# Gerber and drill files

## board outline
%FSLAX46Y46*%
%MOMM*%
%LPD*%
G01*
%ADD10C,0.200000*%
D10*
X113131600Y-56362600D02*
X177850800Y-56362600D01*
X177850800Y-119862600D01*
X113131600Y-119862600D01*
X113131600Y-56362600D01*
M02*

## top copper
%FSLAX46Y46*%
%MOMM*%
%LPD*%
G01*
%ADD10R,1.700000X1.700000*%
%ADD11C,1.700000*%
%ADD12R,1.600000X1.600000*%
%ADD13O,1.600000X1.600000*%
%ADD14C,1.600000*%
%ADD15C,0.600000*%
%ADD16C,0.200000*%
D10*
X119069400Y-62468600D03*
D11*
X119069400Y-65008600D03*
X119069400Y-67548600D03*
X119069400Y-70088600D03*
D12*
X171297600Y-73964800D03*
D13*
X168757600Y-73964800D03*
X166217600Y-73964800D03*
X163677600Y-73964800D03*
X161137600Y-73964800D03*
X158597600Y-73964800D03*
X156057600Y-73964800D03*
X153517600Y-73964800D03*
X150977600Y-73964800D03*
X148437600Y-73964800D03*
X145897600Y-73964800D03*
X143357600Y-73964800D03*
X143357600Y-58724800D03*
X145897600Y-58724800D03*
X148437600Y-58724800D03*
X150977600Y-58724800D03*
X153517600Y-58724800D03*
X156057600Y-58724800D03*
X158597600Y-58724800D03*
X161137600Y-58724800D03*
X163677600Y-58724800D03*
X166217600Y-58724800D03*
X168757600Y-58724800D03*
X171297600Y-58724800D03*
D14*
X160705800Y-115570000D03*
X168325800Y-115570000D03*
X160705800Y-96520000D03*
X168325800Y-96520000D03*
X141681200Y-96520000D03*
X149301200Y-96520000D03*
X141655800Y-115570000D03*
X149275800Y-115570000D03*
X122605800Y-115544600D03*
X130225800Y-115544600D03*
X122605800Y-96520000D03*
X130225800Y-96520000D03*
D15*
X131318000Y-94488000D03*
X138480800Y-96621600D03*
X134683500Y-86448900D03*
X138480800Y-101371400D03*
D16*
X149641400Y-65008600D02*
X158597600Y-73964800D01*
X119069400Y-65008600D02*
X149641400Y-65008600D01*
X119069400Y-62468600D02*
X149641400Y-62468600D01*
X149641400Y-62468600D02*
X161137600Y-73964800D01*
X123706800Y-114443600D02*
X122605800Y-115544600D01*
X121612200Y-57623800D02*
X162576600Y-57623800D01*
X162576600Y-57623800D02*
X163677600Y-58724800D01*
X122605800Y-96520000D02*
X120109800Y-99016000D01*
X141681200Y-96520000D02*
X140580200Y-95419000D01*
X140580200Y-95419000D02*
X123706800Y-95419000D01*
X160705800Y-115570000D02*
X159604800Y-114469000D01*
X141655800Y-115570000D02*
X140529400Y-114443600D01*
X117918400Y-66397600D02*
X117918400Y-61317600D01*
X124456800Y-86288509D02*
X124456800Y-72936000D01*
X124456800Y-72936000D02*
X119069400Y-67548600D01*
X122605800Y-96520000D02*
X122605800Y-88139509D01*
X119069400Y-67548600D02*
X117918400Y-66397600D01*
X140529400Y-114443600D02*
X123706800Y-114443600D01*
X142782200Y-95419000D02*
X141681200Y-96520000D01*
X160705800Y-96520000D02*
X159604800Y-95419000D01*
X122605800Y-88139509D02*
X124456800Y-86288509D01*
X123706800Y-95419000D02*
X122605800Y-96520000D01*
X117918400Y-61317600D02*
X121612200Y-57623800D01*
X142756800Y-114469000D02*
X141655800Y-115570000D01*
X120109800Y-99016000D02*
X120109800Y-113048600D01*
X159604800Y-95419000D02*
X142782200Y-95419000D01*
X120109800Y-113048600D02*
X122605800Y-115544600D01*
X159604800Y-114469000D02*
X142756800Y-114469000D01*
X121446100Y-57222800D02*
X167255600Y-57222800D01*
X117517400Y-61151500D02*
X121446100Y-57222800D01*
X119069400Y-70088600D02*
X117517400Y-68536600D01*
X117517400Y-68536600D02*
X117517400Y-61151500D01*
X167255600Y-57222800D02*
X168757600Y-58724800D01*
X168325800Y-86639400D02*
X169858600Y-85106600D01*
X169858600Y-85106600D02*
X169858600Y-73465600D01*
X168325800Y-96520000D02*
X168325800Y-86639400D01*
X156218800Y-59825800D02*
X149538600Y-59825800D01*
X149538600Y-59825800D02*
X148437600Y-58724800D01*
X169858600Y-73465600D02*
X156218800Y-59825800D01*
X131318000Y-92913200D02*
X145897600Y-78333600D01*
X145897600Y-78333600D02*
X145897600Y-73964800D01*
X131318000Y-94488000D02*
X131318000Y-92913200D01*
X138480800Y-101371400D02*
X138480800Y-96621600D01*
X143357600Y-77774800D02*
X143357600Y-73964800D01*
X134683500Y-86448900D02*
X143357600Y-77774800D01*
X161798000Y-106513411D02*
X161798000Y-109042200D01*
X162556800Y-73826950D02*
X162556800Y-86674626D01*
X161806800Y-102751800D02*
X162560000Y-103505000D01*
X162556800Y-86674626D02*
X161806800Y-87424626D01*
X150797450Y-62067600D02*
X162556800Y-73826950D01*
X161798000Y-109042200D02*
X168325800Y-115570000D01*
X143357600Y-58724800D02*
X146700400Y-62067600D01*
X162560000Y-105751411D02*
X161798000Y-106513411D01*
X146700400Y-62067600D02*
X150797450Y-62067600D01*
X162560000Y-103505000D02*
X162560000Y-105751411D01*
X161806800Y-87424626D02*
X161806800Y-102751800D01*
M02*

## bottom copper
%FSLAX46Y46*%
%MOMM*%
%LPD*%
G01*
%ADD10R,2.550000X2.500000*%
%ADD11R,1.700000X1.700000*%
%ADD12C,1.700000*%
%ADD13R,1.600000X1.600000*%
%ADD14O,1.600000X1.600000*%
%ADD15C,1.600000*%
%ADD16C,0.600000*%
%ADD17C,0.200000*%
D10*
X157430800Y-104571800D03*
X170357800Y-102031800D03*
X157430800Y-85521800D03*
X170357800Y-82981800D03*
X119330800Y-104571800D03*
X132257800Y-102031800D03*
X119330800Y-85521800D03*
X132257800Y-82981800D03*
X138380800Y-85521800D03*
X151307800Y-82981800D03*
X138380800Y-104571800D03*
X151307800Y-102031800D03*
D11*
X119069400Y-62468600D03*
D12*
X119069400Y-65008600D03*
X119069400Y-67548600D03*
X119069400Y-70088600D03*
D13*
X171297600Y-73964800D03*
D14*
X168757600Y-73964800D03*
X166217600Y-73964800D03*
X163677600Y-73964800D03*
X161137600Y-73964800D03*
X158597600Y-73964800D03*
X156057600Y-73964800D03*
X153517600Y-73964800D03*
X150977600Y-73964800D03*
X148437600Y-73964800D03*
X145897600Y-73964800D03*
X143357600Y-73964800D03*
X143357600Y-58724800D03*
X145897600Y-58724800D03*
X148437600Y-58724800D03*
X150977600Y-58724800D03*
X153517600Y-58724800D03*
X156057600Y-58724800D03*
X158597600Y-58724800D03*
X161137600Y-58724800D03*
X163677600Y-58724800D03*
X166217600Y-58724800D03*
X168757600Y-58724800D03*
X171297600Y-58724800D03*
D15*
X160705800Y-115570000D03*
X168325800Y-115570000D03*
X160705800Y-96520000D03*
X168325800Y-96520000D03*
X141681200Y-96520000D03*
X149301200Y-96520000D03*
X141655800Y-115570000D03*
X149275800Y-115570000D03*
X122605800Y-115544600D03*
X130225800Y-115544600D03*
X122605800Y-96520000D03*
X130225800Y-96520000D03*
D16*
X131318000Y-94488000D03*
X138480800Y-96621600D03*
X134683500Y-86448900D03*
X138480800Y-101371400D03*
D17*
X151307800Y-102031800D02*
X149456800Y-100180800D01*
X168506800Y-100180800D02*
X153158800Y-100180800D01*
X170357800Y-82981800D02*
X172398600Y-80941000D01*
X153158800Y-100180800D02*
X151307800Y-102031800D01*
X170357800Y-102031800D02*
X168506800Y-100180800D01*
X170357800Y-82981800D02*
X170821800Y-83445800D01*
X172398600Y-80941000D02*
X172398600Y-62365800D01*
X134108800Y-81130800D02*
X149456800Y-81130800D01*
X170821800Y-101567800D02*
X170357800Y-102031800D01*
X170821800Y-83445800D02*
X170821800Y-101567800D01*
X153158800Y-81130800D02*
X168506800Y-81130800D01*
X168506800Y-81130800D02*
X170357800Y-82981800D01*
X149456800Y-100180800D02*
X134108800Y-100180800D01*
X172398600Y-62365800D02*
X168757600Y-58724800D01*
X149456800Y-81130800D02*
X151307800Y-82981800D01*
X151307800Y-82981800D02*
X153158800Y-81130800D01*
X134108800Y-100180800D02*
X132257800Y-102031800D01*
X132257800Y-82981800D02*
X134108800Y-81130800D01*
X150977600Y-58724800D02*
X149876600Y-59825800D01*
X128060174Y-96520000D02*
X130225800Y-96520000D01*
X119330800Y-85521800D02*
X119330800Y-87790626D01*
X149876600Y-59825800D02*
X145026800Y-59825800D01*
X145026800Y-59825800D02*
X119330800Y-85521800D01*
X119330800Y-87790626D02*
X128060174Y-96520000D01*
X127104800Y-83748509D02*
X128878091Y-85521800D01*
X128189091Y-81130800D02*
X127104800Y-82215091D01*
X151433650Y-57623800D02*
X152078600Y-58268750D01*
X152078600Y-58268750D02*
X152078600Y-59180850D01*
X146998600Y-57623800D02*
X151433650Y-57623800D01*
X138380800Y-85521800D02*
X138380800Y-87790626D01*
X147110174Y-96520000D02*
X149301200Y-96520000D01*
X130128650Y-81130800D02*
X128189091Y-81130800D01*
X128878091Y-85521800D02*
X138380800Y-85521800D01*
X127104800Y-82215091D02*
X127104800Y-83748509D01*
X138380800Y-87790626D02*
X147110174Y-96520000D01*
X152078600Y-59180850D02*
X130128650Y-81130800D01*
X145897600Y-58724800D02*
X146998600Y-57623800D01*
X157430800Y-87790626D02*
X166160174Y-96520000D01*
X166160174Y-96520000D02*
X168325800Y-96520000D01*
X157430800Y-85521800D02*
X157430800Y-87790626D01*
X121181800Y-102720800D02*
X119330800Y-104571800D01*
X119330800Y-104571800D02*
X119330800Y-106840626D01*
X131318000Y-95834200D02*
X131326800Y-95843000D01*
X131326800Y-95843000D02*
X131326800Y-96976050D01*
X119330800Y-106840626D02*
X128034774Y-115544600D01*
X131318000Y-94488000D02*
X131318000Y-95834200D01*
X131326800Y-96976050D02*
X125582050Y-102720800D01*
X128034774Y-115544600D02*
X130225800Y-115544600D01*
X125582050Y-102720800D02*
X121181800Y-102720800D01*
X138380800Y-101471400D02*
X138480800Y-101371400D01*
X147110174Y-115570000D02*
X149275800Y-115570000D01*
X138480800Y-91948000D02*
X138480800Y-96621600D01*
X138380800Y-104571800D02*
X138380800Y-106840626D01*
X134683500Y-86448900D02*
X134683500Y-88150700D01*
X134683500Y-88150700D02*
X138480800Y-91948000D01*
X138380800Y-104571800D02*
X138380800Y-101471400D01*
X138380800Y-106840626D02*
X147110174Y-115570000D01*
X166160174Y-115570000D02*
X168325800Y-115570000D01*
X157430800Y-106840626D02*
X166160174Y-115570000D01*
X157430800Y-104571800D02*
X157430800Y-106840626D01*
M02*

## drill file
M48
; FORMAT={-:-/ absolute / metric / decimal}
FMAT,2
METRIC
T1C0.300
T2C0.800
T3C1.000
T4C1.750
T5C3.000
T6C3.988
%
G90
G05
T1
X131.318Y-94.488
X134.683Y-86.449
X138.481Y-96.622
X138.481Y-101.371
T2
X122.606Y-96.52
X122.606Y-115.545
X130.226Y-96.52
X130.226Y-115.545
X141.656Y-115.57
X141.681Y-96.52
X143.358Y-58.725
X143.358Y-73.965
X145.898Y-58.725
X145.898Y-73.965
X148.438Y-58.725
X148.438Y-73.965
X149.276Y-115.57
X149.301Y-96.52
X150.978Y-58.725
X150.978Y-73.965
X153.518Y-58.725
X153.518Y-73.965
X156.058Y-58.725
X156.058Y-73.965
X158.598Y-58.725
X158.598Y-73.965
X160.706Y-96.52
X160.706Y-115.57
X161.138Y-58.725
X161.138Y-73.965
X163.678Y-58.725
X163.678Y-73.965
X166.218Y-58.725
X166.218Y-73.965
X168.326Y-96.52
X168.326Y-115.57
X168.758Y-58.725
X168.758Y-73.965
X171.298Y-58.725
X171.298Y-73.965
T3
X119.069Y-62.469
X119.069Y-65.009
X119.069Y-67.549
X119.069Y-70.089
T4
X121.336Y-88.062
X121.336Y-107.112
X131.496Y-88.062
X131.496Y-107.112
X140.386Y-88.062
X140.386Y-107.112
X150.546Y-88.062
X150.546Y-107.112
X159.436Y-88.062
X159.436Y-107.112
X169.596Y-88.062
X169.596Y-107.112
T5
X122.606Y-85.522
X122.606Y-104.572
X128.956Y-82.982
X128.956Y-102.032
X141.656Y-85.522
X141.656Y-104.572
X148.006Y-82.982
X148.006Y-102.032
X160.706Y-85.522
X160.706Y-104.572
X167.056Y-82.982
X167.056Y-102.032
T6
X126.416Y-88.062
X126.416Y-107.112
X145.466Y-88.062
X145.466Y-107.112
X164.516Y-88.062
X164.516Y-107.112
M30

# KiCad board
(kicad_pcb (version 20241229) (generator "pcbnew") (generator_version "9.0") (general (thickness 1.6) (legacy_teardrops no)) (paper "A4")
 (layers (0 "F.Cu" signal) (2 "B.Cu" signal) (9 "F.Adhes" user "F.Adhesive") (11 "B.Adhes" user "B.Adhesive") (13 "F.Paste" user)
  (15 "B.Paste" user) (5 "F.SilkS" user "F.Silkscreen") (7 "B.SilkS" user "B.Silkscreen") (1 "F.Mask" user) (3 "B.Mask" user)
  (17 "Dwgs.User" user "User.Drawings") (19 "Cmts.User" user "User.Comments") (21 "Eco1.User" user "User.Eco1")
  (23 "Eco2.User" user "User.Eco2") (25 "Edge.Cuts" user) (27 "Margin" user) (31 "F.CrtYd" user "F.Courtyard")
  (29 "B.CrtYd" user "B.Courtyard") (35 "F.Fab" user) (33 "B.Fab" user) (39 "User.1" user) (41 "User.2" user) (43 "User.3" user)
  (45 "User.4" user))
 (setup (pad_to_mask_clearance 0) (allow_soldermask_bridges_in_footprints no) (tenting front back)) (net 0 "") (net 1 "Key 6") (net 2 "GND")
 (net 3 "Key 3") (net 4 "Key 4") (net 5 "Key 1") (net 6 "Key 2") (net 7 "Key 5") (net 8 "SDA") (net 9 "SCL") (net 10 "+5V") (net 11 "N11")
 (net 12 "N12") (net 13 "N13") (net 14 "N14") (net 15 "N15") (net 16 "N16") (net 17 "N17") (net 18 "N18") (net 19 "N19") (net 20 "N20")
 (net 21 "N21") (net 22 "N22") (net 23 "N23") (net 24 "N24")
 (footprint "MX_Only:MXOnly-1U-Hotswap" (layer "F.Cu") (at 164.5158 107.1118)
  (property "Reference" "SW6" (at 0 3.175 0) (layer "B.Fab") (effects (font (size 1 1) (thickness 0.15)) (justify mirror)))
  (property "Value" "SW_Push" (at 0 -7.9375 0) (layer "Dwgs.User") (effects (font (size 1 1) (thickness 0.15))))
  (pad "" np_thru_hole circle (at -5.08 0 48.0996) (size 1.75 1.75) (drill 1.75) (layers "*.Cu" "*.Mask"))
  (pad "" np_thru_hole circle (at -3.81 -2.54) (size 3 3) (drill 3) (layers "*.Cu" "*.Mask"))
  (pad "" np_thru_hole circle (at 0 0) (size 3.9878 3.9878) (drill 3.9878) (layers "*.Cu" "*.Mask"))
  (pad "" np_thru_hole circle (at 2.54 -5.08) (size 3 3) (drill 3) (layers "*.Cu" "*.Mask"))
  (pad "" np_thru_hole circle (at 5.08 0 48.0996) (size 1.75 1.75) (drill 1.75) (layers "*.Cu" "*.Mask"))
  (pad "1" smd rect (at -7.085 -2.54) (size 2.55 2.5) (layers "B.Cu" "B.Mask" "B.Paste") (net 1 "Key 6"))
  (pad "2" smd rect (at 5.842 -5.08) (size 2.55 2.5) (layers "B.Cu" "B.Mask" "B.Paste") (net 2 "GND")))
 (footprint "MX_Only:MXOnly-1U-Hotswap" (layer "F.Cu") (at 164.5158 88.0618)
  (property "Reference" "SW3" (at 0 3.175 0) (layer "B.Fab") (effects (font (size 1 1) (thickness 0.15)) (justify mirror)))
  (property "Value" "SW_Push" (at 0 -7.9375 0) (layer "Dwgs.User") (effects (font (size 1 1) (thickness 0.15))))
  (pad "" np_thru_hole circle (at -5.08 0 48.0996) (size 1.75 1.75) (drill 1.75) (layers "*.Cu" "*.Mask"))
  (pad "" np_thru_hole circle (at -3.81 -2.54) (size 3 3) (drill 3) (layers "*.Cu" "*.Mask"))
  (pad "" np_thru_hole circle (at 0 0) (size 3.9878 3.9878) (drill 3.9878) (layers "*.Cu" "*.Mask"))
  (pad "" np_thru_hole circle (at 2.54 -5.08) (size 3 3) (drill 3) (layers "*.Cu" "*.Mask"))
  (pad "" np_thru_hole circle (at 5.08 0 48.0996) (size 1.75 1.75) (drill 1.75) (layers "*.Cu" "*.Mask"))
  (pad "1" smd rect (at -7.085 -2.54) (size 2.55 2.5) (layers "B.Cu" "B.Mask" "B.Paste") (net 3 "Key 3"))
  (pad "2" smd rect (at 5.842 -5.08) (size 2.55 2.5) (layers "B.Cu" "B.Mask" "B.Paste") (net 2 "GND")))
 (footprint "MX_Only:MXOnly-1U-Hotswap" (layer "F.Cu") (at 126.4158 107.1118)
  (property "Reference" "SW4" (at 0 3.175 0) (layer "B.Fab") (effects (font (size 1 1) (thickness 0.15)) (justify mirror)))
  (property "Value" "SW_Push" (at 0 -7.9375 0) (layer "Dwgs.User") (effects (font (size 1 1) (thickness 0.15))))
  (pad "" np_thru_hole circle (at -5.08 0 48.0996) (size 1.75 1.75) (drill 1.75) (layers "*.Cu" "*.Mask"))
  (pad "" np_thru_hole circle (at -3.81 -2.54) (size 3 3) (drill 3) (layers "*.Cu" "*.Mask"))
  (pad "" np_thru_hole circle (at 0 0) (size 3.9878 3.9878) (drill 3.9878) (layers "*.Cu" "*.Mask"))
  (pad "" np_thru_hole circle (at 2.54 -5.08) (size 3 3) (drill 3) (layers "*.Cu" "*.Mask"))
  (pad "" np_thru_hole circle (at 5.08 0 48.0996) (size 1.75 1.75) (drill 1.75) (layers "*.Cu" "*.Mask"))
  (pad "1" smd rect (at -7.085 -2.54) (size 2.55 2.5) (layers "B.Cu" "B.Mask" "B.Paste") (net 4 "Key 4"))
  (pad "2" smd rect (at 5.842 -5.08) (size 2.55 2.5) (layers "B.Cu" "B.Mask" "B.Paste") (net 2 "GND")))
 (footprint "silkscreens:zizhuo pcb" (layer "F.Cu") (at 164.6936 67.346207 90)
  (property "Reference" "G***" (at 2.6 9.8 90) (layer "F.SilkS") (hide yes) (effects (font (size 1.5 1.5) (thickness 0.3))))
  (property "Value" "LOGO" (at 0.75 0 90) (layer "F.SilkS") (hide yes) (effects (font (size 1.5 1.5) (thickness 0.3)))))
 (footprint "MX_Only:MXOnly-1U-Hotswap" (layer "F.Cu") (at 126.4158 88.0618)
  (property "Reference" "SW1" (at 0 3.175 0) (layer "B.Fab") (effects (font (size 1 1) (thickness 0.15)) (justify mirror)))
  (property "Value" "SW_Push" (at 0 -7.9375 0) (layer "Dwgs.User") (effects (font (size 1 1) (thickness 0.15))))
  (pad "" np_thru_hole circle (at -5.08 0 48.0996) (size 1.75 1.75) (drill 1.75) (layers "*.Cu" "*.Mask"))
  (pad "" np_thru_hole circle (at -3.81 -2.54) (size 3 3) (drill 3) (layers "*.Cu" "*.Mask"))
  (pad "" np_thru_hole circle (at 0 0) (size 3.9878 3.9878) (drill 3.9878) (layers "*.Cu" "*.Mask"))
  (pad "" np_thru_hole circle (at 2.54 -5.08) (size 3 3) (drill 3) (layers "*.Cu" "*.Mask"))
  (pad "" np_thru_hole circle (at 5.08 0 48.0996) (size 1.75 1.75) (drill 1.75) (layers "*.Cu" "*.Mask"))
  (pad "1" smd rect (at -7.085 -2.54) (size 2.55 2.5) (layers "B.Cu" "B.Mask" "B.Paste") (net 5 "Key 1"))
  (pad "2" smd rect (at 5.842 -5.08) (size 2.55 2.5) (layers "B.Cu" "B.Mask" "B.Paste") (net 2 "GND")))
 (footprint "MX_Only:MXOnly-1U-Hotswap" (layer "F.Cu") (at 145.4658 88.0618)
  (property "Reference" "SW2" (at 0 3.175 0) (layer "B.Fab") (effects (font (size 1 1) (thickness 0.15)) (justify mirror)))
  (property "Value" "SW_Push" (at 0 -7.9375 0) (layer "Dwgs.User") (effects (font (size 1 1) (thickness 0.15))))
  (pad "" np_thru_hole circle (at -5.08 0 48.0996) (size 1.75 1.75) (drill 1.75) (layers "*.Cu" "*.Mask"))
  (pad "" np_thru_hole circle (at -3.81 -2.54) (size 3 3) (drill 3) (layers "*.Cu" "*.Mask"))
  (pad "" np_thru_hole circle (at 0 0) (size 3.9878 3.9878) (drill 3.9878) (layers "*.Cu" "*.Mask"))
  (pad "" np_thru_hole circle (at 2.54 -5.08) (size 3 3) (drill 3) (layers "*.Cu" "*.Mask"))
  (pad "" np_thru_hole circle (at 5.08 0 48.0996) (size 1.75 1.75) (drill 1.75) (layers "*.Cu" "*.Mask"))
  (pad "1" smd rect (at -7.085 -2.54) (size 2.55 2.5) (layers "B.Cu" "B.Mask" "B.Paste") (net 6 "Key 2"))
  (pad "2" smd rect (at 5.842 -5.08) (size 2.55 2.5) (layers "B.Cu" "B.Mask" "B.Paste") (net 2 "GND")))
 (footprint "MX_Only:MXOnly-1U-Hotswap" (layer "F.Cu") (at 145.4658 107.1118)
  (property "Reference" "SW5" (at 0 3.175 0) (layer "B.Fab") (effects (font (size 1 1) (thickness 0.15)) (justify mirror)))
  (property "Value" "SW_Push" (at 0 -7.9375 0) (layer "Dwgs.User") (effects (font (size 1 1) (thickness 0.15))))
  (pad "" np_thru_hole circle (at -5.08 0 48.0996) (size 1.75 1.75) (drill 1.75) (layers "*.Cu" "*.Mask"))
  (pad "" np_thru_hole circle (at -3.81 -2.54) (size 3 3) (drill 3) (layers "*.Cu" "*.Mask"))
  (pad "" np_thru_hole circle (at 0 0) (size 3.9878 3.9878) (drill 3.9878) (layers "*.Cu" "*.Mask"))
  (pad "" np_thru_hole circle (at 2.54 -5.08) (size 3 3) (drill 3) (layers "*.Cu" "*.Mask"))
  (pad "" np_thru_hole circle (at 5.08 0 48.0996) (size 1.75 1.75) (drill 1.75) (layers "*.Cu" "*.Mask"))
  (pad "1" smd rect (at -7.085 -2.54) (size 2.55 2.5) (layers "B.Cu" "B.Mask" "B.Paste") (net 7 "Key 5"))
  (pad "2" smd rect (at 5.842 -5.08) (size 2.55 2.5) (layers "B.Cu" "B.Mask" "B.Paste") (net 2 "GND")))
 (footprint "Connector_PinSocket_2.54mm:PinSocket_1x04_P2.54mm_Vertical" (layer "F.Cu") (at 119.0694 62.4686)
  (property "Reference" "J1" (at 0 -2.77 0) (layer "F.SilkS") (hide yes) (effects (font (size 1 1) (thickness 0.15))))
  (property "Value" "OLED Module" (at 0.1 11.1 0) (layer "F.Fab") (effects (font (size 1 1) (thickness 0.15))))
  (pad "1" thru_hole rect (at 0 0) (size 1.7 1.7) (drill 1) (layers "*.Cu" "*.Mask") (remove_unused_layers no) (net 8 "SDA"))
  (pad "2" thru_hole circle (at 0 2.54) (size 1.7 1.7) (drill 1) (layers "*.Cu" "*.Mask") (remove_unused_layers no) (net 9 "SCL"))
  (pad "3" thru_hole circle (at 0 5.08) (size 1.7 1.7) (drill 1) (layers "*.Cu" "*.Mask") (remove_unused_layers no) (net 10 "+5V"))
  (pad "4" thru_hole circle (at 0 7.62) (size 1.7 1.7) (drill 1) (layers "*.Cu" "*.Mask") (remove_unused_layers no) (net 2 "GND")))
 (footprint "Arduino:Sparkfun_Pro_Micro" (layer "B.Cu") (at 143.3576 58.7248 -90)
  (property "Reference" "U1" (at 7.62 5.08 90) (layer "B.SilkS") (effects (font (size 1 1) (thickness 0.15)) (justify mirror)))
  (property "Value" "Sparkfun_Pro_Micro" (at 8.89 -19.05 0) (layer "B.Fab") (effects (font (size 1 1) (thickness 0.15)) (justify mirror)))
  (pad "1" thru_hole rect (at 15.24 -27.94 270) (size 1.6 1.6) (drill 0.8) (layers "*.Cu" "*.Mask") (remove_unused_layers no) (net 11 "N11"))
  (pad "2" thru_hole oval (at 15.24 -25.4 270) (size 1.6 1.6) (drill 0.8) (layers "*.Cu" "*.Mask") (remove_unused_layers no) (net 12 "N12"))
  (pad "3" thru_hole oval (at 15.24 -22.86 270) (size 1.6 1.6) (drill 0.8) (layers "*.Cu" "*.Mask") (remove_unused_layers no) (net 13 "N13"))
  (pad "4" thru_hole oval (at 15.24 -20.32 270) (size 1.6 1.6) (drill 0.8) (layers "*.Cu" "*.Mask") (remove_unused_layers no) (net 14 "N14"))
  (pad "5" thru_hole oval (at 15.24 -17.78 270) (size 1.6 1.6) (drill 0.8) (layers "*.Cu" "*.Mask") (remove_unused_layers no) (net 8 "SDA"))
  (pad "6" thru_hole oval (at 15.24 -15.24 270) (size 1.6 1.6) (drill 0.8) (layers "*.Cu" "*.Mask") (remove_unused_layers no) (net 9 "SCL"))
  (pad "7" thru_hole oval (at 15.24 -12.7 270) (size 1.6 1.6) (drill 0.8) (layers "*.Cu" "*.Mask") (remove_unused_layers no) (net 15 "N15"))
  (pad "8" thru_hole oval (at 15.24 -10.16 270) (size 1.6 1.6) (drill 0.8) (layers "*.Cu" "*.Mask") (remove_unused_layers no) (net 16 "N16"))
  (pad "9" thru_hole oval (at 15.24 -7.62 270) (size 1.6 1.6) (drill 0.8) (layers "*.Cu" "*.Mask") (remove_unused_layers no) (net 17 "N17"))
  (pad "10" thru_hole oval (at 15.24 -5.08 270) (size 1.6 1.6) (drill 0.8) (layers "*.Cu" "*.Mask") (remove_unused_layers no) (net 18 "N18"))
  (pad "11" thru_hole oval (at 15.24 -2.54 270) (size 1.6 1.6) (drill 0.8) (layers "*.Cu" "*.Mask") (remove_unused_layers no)
   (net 4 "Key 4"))
  (pad "12" thru_hole oval (at 15.24 0 270) (size 1.6 1.6) (drill 0.8) (layers "*.Cu" "*.Mask") (remove_unused_layers no) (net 7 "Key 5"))
  (pad "13" thru_hole oval (at 0 0 270) (size 1.6 1.6) (drill 0.8) (layers "*.Cu" "*.Mask") (remove_unused_layers no) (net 1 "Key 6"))
  (pad "14" thru_hole oval (at 0 -2.54 270) (size 1.6 1.6) (drill 0.8) (layers "*.Cu" "*.Mask") (remove_unused_layers no) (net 6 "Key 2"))
  (pad "15" thru_hole oval (at 0 -5.08 270) (size 1.6 1.6) (drill 0.8) (layers "*.Cu" "*.Mask") (remove_unused_layers no) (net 3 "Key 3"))
  (pad "16" thru_hole oval (at 0 -7.62 270) (size 1.6 1.6) (drill 0.8) (layers "*.Cu" "*.Mask") (remove_unused_layers no) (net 5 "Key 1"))
  (pad "17" thru_hole oval (at 0 -10.16 270) (size 1.6 1.6) (drill 0.8) (layers "*.Cu" "*.Mask") (remove_unused_layers no) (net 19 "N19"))
  (pad "18" thru_hole oval (at 0 -12.7 270) (size 1.6 1.6) (drill 0.8) (layers "*.Cu" "*.Mask") (remove_unused_layers no) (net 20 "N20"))
  (pad "19" thru_hole oval (at 0 -15.24 270) (size 1.6 1.6) (drill 0.8) (layers "*.Cu" "*.Mask") (remove_unused_layers no) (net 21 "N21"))
  (pad "20" thru_hole oval (at 0 -17.78 270) (size 1.6 1.6) (drill 0.8) (layers "*.Cu" "*.Mask") (remove_unused_layers no) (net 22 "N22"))
  (pad "21" thru_hole oval (at 0 -20.32 270) (size 1.6 1.6) (drill 0.8) (layers "*.Cu" "*.Mask") (remove_unused_layers no) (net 10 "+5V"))
  (pad "22" thru_hole oval (at 0 -22.86 270) (size 1.6 1.6) (drill 0.8) (layers "*.Cu" "*.Mask") (remove_unused_layers no) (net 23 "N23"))
  (pad "23" thru_hole oval (at 0 -25.4 270) (size 1.6 1.6) (drill 0.8) (layers "*.Cu" "*.Mask") (remove_unused_layers no) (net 2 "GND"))
  (pad "24" thru_hole oval (at 0 -27.94 270) (size 1.6 1.6) (drill 0.8) (layers "*.Cu" "*.Mask") (remove_unused_layers no) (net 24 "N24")))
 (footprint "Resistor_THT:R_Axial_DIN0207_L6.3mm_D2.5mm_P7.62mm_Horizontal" (layer "B.Cu") (at 160.7058 115.57)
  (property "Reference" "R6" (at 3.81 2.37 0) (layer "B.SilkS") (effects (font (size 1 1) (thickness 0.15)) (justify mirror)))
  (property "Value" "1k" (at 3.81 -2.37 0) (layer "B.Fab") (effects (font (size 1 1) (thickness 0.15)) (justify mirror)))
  (pad "1" thru_hole circle (at 0 0) (size 1.6 1.6) (drill 0.8) (layers "*.Cu" "*.Mask") (remove_unused_layers no) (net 10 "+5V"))
  (pad "2" thru_hole circle (at 7.62 0) (size 1.6 1.6) (drill 0.8) (layers "*.Cu" "*.Mask") (remove_unused_layers no) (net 1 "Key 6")))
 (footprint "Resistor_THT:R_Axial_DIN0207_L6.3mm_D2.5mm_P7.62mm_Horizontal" (layer "B.Cu") (at 160.7058 96.52)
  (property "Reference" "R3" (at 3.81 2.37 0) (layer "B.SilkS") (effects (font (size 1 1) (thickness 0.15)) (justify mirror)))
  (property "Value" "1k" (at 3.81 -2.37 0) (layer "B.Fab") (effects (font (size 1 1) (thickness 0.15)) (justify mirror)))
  (pad "1" thru_hole circle (at 0 0) (size 1.6 1.6) (drill 0.8) (layers "*.Cu" "*.Mask") (remove_unused_layers no) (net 10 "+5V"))
  (pad "2" thru_hole circle (at 7.62 0) (size 1.6 1.6) (drill 0.8) (layers "*.Cu" "*.Mask") (remove_unused_layers no) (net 3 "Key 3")))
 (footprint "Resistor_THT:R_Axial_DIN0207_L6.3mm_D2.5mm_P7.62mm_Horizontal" (layer "B.Cu") (at 141.6812 96.52)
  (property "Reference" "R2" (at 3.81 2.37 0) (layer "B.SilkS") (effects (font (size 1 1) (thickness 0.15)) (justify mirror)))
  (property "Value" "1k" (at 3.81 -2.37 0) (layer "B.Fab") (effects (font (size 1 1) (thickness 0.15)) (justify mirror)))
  (pad "1" thru_hole circle (at 0 0) (size 1.6 1.6) (drill 0.8) (layers "*.Cu" "*.Mask") (remove_unused_layers no) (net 10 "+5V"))
  (pad "2" thru_hole circle (at 7.62 0) (size 1.6 1.6) (drill 0.8) (layers "*.Cu" "*.Mask") (remove_unused_layers no) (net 6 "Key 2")))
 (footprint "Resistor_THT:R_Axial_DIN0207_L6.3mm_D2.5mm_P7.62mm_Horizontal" (layer "B.Cu") (at 141.6558 115.57)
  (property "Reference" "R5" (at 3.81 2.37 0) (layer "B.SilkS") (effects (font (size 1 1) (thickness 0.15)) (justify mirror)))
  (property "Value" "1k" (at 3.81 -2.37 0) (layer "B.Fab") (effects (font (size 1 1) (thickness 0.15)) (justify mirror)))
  (pad "1" thru_hole circle (at 0 0) (size 1.6 1.6) (drill 0.8) (layers "*.Cu" "*.Mask") (remove_unused_layers no) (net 10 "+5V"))
  (pad "2" thru_hole circle (at 7.62 0) (size 1.6 1.6) (drill 0.8) (layers "*.Cu" "*.Mask") (remove_unused_layers no) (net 7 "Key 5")))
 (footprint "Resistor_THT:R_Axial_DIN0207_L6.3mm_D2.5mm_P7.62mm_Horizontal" (layer "B.Cu") (at 122.6058 115.5446)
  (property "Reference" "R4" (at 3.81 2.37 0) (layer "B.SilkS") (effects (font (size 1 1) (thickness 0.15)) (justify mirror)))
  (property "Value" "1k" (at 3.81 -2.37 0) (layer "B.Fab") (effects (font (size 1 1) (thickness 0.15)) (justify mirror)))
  (pad "1" thru_hole circle (at 0 0) (size 1.6 1.6) (drill 0.8) (layers "*.Cu" "*.Mask") (remove_unused_layers no) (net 10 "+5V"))
  (pad "2" thru_hole circle (at 7.62 0) (size 1.6 1.6) (drill 0.8) (layers "*.Cu" "*.Mask") (remove_unused_layers no) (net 4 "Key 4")))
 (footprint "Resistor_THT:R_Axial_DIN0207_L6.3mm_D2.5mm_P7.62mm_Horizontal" (layer "B.Cu") (at 122.6058 96.52)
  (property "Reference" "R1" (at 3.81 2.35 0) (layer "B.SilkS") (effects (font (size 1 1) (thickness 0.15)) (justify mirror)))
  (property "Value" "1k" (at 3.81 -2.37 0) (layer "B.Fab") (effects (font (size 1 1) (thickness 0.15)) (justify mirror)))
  (pad "1" thru_hole circle (at 0 0) (size 1.6 1.6) (drill 0.8) (layers "*.Cu" "*.Mask") (remove_unused_layers no) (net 10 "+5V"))
  (pad "2" thru_hole circle (at 7.62 0) (size 1.6 1.6) (drill 0.8) (layers "*.Cu" "*.Mask") (remove_unused_layers no) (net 5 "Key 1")))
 (gr_rect (start 113.1316 56.3626) (end 177.8508 119.8626) (stroke (width 0.2) (type solid)) (fill no) (layer "Edge.Cuts"))
 (segment (start 149.6414 65.0086) (end 158.5976 73.9648) (width 0.2) (layer "F.Cu") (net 9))
 (segment (start 119.0694 65.0086) (end 149.6414 65.0086) (width 0.2) (layer "F.Cu") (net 9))
 (segment (start 119.0694 62.4686) (end 149.6414 62.4686) (width 0.2) (layer "F.Cu") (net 8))
 (segment (start 149.6414 62.4686) (end 161.1376 73.9648) (width 0.2) (layer "F.Cu") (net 8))
 (segment (start 123.7068 114.4436) (end 122.6058 115.5446) (width 0.2) (layer "F.Cu") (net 10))
 (segment (start 121.6122 57.6238) (end 162.5766 57.6238) (width 0.2) (layer "F.Cu") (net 10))
 (segment (start 162.5766 57.6238) (end 163.6776 58.7248) (width 0.2) (layer "F.Cu") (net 10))
 (segment (start 122.6058 96.52) (end 120.1098 99.016) (width 0.2) (layer "F.Cu") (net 10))
 (segment (start 141.6812 96.52) (end 140.5802 95.419) (width 0.2) (layer "F.Cu") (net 10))
 (segment (start 140.5802 95.419) (end 123.7068 95.419) (width 0.2) (layer "F.Cu") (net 10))
 (segment (start 160.7058 115.57) (end 159.6048 114.469) (width 0.2) (layer "F.Cu") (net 10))
 (segment (start 141.6558 115.57) (end 140.5294 114.4436) (width 0.2) (layer "F.Cu") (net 10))
 (segment (start 117.9184 66.3976) (end 117.9184 61.3176) (width 0.2) (layer "F.Cu") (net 10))
 (segment (start 124.4568 86.288509) (end 124.4568 72.936) (width 0.2) (layer "F.Cu") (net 10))
 (segment (start 124.4568 72.936) (end 119.0694 67.5486) (width 0.2) (layer "F.Cu") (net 10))
 (segment (start 122.6058 96.52) (end 122.6058 88.139509) (width 0.2) (layer "F.Cu") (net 10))
 (segment (start 119.0694 67.5486) (end 117.9184 66.3976) (width 0.2) (layer "F.Cu") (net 10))
 (segment (start 140.5294 114.4436) (end 123.7068 114.4436) (width 0.2) (layer "F.Cu") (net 10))
 (segment (start 142.7822 95.419) (end 141.6812 96.52) (width 0.2) (layer "F.Cu") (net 10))
 (segment (start 160.7058 96.52) (end 159.6048 95.419) (width 0.2) (layer "F.Cu") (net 10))
 (segment (start 122.6058 88.139509) (end 124.4568 86.288509) (width 0.2) (layer "F.Cu") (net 10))
 (segment (start 123.7068 95.419) (end 122.6058 96.52) (width 0.2) (layer "F.Cu") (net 10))
 (segment (start 117.9184 61.3176) (end 121.6122 57.6238) (width 0.2) (layer "F.Cu") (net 10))
 (segment (start 142.7568 114.469) (end 141.6558 115.57) (width 0.2) (layer "F.Cu") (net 10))
 (segment (start 120.1098 99.016) (end 120.1098 113.0486) (width 0.2) (layer "F.Cu") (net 10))
 (segment (start 159.6048 95.419) (end 142.7822 95.419) (width 0.2) (layer "F.Cu") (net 10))
 (segment (start 120.1098 113.0486) (end 122.6058 115.5446) (width 0.2) (layer "F.Cu") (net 10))
 (segment (start 159.6048 114.469) (end 142.7568 114.469) (width 0.2) (layer "F.Cu") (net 10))
 (segment (start 121.4461 57.2228) (end 167.2556 57.2228) (width 0.2) (layer "F.Cu") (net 2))
 (segment (start 117.5174 61.1515) (end 121.4461 57.2228) (width 0.2) (layer "F.Cu") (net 2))
 (segment (start 119.0694 70.0886) (end 117.5174 68.5366) (width 0.2) (layer "F.Cu") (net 2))
 (segment (start 117.5174 68.5366) (end 117.5174 61.1515) (width 0.2) (layer "F.Cu") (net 2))
 (segment (start 167.2556 57.2228) (end 168.7576 58.7248) (width 0.2) (layer "F.Cu") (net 2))
 (segment (start 151.3078 102.0318) (end 149.4568 100.1808) (width 0.2) (layer "B.Cu") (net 2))
 (segment (start 168.5068 100.1808) (end 153.1588 100.1808) (width 0.2) (layer "B.Cu") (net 2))
 (segment (start 170.3578 82.9818) (end 172.3986 80.941) (width 0.2) (layer "B.Cu") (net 2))
 (segment (start 153.1588 100.1808) (end 151.3078 102.0318) (width 0.2) (layer "B.Cu") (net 2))
 (segment (start 170.3578 102.0318) (end 168.5068 100.1808) (width 0.2) (layer "B.Cu") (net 2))
 (segment (start 170.3578 82.9818) (end 170.8218 83.4458) (width 0.2) (layer "B.Cu") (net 2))
 (segment (start 172.3986 80.941) (end 172.3986 62.3658) (width 0.2) (layer "B.Cu") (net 2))
 (segment (start 134.1088 81.1308) (end 149.4568 81.1308) (width 0.2) (layer "B.Cu") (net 2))
 (segment (start 170.8218 101.5678) (end 170.3578 102.0318) (width 0.2) (layer "B.Cu") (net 2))
 (segment (start 170.8218 83.4458) (end 170.8218 101.5678) (width 0.2) (layer "B.Cu") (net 2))
 (segment (start 153.1588 81.1308) (end 168.5068 81.1308) (width 0.2) (layer "B.Cu") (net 2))
 (segment (start 168.5068 81.1308) (end 170.3578 82.9818) (width 0.2) (layer "B.Cu") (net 2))
 (segment (start 149.4568 100.1808) (end 134.1088 100.1808) (width 0.2) (layer "B.Cu") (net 2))
 (segment (start 172.3986 62.3658) (end 168.7576 58.7248) (width 0.2) (layer "B.Cu") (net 2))
 (segment (start 149.4568 81.1308) (end 151.3078 82.9818) (width 0.2) (layer "B.Cu") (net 2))
 (segment (start 151.3078 82.9818) (end 153.1588 81.1308) (width 0.2) (layer "B.Cu") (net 2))
 (segment (start 134.1088 100.1808) (end 132.2578 102.0318) (width 0.2) (layer "B.Cu") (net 2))
 (segment (start 132.2578 82.9818) (end 134.1088 81.1308) (width 0.2) (layer "B.Cu") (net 2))
 (segment (start 150.9776 58.7248) (end 149.8766 59.8258) (width 0.2) (layer "B.Cu") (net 5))
 (segment (start 128.060174 96.52) (end 130.2258 96.52) (width 0.2) (layer "B.Cu") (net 5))
 (segment (start 119.3308 85.5218) (end 119.3308 87.790626) (width 0.2) (layer "B.Cu") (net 5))
 (segment (start 149.8766 59.8258) (end 145.0268 59.8258) (width 0.2) (layer "B.Cu") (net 5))
 (segment (start 145.0268 59.8258) (end 119.3308 85.5218) (width 0.2) (layer "B.Cu") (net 5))
 (segment (start 119.3308 87.790626) (end 128.060174 96.52) (width 0.2) (layer "B.Cu") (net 5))
 (segment (start 127.1048 83.748509) (end 128.878091 85.5218) (width 0.2) (layer "B.Cu") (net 6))
 (segment (start 128.189091 81.1308) (end 127.1048 82.215091) (width 0.2) (layer "B.Cu") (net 6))
 (segment (start 151.43365 57.6238) (end 152.0786 58.26875) (width 0.2) (layer "B.Cu") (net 6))
 (segment (start 152.0786 58.26875) (end 152.0786 59.18085) (width 0.2) (layer "B.Cu") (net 6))
 (segment (start 146.9986 57.6238) (end 151.43365 57.6238) (width 0.2) (layer "B.Cu") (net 6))
 (segment (start 138.3808 85.5218) (end 138.3808 87.790626) (width 0.2) (layer "B.Cu") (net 6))
 (segment (start 147.110174 96.52) (end 149.3012 96.52) (width 0.2) (layer "B.Cu") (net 6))
 (segment (start 130.12865 81.1308) (end 128.189091 81.1308) (width 0.2) (layer "B.Cu") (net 6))
 (segment (start 128.878091 85.5218) (end 138.3808 85.5218) (width 0.2) (layer "B.Cu") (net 6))
 (segment (start 127.1048 82.215091) (end 127.1048 83.748509) (width 0.2) (layer "B.Cu") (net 6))
 (segment (start 138.3808 87.790626) (end 147.110174 96.52) (width 0.2) (layer "B.Cu") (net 6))
 (segment (start 152.0786 59.18085) (end 130.12865 81.1308) (width 0.2) (layer "B.Cu") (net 6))
 (segment (start 145.8976 58.7248) (end 146.9986 57.6238) (width 0.2) (layer "B.Cu") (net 6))
 (segment (start 168.3258 86.6394) (end 169.8586 85.1066) (width 0.2) (layer "F.Cu") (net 3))
 (segment (start 169.8586 85.1066) (end 169.8586 73.4656) (width 0.2) (layer "F.Cu") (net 3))
 (segment (start 168.3258 96.52) (end 168.3258 86.6394) (width 0.2) (layer "F.Cu") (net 3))
 (segment (start 156.2188 59.8258) (end 149.5386 59.8258) (width 0.2) (layer "F.Cu") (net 3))
 (segment (start 149.5386 59.8258) (end 148.4376 58.7248) (width 0.2) (layer "F.Cu") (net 3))
 (segment (start 169.8586 73.4656) (end 156.2188 59.8258) (width 0.2) (layer "F.Cu") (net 3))
 (segment (start 157.4308 87.790626) (end 166.160174 96.52) (width 0.2) (layer "B.Cu") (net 3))
 (segment (start 166.160174 96.52) (end 168.3258 96.52) (width 0.2) (layer "B.Cu") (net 3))
 (segment (start 157.4308 85.5218) (end 157.4308 87.790626) (width 0.2) (layer "B.Cu") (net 3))
 (segment (start 131.318 92.9132) (end 145.8976 78.3336) (width 0.2) (layer "F.Cu") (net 4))
 (segment (start 145.8976 78.3336) (end 145.8976 73.9648) (width 0.2) (layer "F.Cu") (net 4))
 (segment (start 131.318 94.488) (end 131.318 92.9132) (width 0.2) (layer "F.Cu") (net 4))
 (via (at 131.318 94.488) (size 0.6) (drill 0.3) (layers "F.Cu" "B.Cu") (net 4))
 (segment (start 121.1818 102.7208) (end 119.3308 104.5718) (width 0.2) (layer "B.Cu") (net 4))
 (segment (start 119.3308 104.5718) (end 119.3308 106.840626) (width 0.2) (layer "B.Cu") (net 4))
 (segment (start 131.318 95.8342) (end 131.3268 95.843) (width 0.2) (layer "B.Cu") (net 4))
 (segment (start 131.3268 95.843) (end 131.3268 96.97605) (width 0.2) (layer "B.Cu") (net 4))
 (segment (start 119.3308 106.840626) (end 128.034774 115.5446) (width 0.2) (layer "B.Cu") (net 4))
 (segment (start 131.318 94.488) (end 131.318 95.8342) (width 0.2) (layer "B.Cu") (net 4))
 (segment (start 131.3268 96.97605) (end 125.58205 102.7208) (width 0.2) (layer "B.Cu") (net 4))
 (segment (start 128.034774 115.5446) (end 130.2258 115.5446) (width 0.2) (layer "B.Cu") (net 4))
 (segment (start 125.58205 102.7208) (end 121.1818 102.7208) (width 0.2) (layer "B.Cu") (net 4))
 (segment (start 138.4808 101.3714) (end 138.4808 96.6216) (width 0.2) (layer "F.Cu") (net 7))
 (segment (start 143.3576 77.7748) (end 143.3576 73.9648) (width 0.2) (layer "F.Cu") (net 7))
 (segment (start 134.6835 86.4489) (end 143.3576 77.7748) (width 0.2) (layer "F.Cu") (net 7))
 (via (at 138.4808 96.6216) (size 0.6) (drill 0.3) (layers "F.Cu" "B.Cu") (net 7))
 (via (at 134.6835 86.4489) (size 0.6) (drill 0.3) (layers "F.Cu" "B.Cu") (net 7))
 (via (at 138.4808 101.3714) (size 0.6) (drill 0.3) (layers "F.Cu" "B.Cu") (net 7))
 (segment (start 138.3808 101.4714) (end 138.4808 101.3714) (width 0.2) (layer "B.Cu") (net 7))
 (segment (start 147.110174 115.57) (end 149.2758 115.57) (width 0.2) (layer "B.Cu") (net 7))
 (segment (start 138.4808 91.948) (end 138.4808 96.6216) (width 0.2) (layer "B.Cu") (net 7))
 (segment (start 138.3808 104.5718) (end 138.3808 106.840626) (width 0.2) (layer "B.Cu") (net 7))
 (segment (start 134.6835 86.4489) (end 134.6835 88.1507) (width 0.2) (layer "B.Cu") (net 7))
 (segment (start 134.6835 88.1507) (end 138.4808 91.948) (width 0.2) (layer "B.Cu") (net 7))
 (segment (start 138.3808 104.5718) (end 138.3808 101.4714) (width 0.2) (layer "B.Cu") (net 7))
 (segment (start 138.3808 106.840626) (end 147.110174 115.57) (width 0.2) (layer "B.Cu") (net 7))
 (segment (start 161.798 106.513411) (end 161.798 109.0422) (width 0.2) (layer "F.Cu") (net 1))
 (segment (start 162.5568 73.82695) (end 162.5568 86.674626) (width 0.2) (layer "F.Cu") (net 1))
 (segment (start 161.8068 102.7518) (end 162.56 103.505) (width 0.2) (layer "F.Cu") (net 1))
 (segment (start 162.5568 86.674626) (end 161.8068 87.424626) (width 0.2) (layer "F.Cu") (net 1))
 (segment (start 150.79745 62.0676) (end 162.5568 73.82695) (width 0.2) (layer "F.Cu") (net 1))
 (segment (start 161.798 109.0422) (end 168.3258 115.57) (width 0.2) (layer "F.Cu") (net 1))
 (segment (start 143.3576 58.7248) (end 146.7004 62.0676) (width 0.2) (layer "F.Cu") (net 1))
 (segment (start 162.56 105.751411) (end 161.798 106.513411) (width 0.2) (layer "F.Cu") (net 1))
 (segment (start 146.7004 62.0676) (end 150.79745 62.0676) (width 0.2) (layer "F.Cu") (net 1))
 (segment (start 162.56 103.505) (end 162.56 105.751411) (width 0.2) (layer "F.Cu") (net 1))
 (segment (start 161.8068 87.424626) (end 161.8068 102.7518) (width 0.2) (layer "F.Cu") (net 1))
 (segment (start 166.160174 115.57) (end 168.3258 115.57) (width 0.2) (layer "B.Cu") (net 1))
 (segment (start 157.4308 106.840626) (end 166.160174 115.57) (width 0.2) (layer "B.Cu") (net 1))
 (segment (start 157.4308 104.5718) (end 157.4308 106.840626) (width 0.2) (layer "B.Cu") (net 1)))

